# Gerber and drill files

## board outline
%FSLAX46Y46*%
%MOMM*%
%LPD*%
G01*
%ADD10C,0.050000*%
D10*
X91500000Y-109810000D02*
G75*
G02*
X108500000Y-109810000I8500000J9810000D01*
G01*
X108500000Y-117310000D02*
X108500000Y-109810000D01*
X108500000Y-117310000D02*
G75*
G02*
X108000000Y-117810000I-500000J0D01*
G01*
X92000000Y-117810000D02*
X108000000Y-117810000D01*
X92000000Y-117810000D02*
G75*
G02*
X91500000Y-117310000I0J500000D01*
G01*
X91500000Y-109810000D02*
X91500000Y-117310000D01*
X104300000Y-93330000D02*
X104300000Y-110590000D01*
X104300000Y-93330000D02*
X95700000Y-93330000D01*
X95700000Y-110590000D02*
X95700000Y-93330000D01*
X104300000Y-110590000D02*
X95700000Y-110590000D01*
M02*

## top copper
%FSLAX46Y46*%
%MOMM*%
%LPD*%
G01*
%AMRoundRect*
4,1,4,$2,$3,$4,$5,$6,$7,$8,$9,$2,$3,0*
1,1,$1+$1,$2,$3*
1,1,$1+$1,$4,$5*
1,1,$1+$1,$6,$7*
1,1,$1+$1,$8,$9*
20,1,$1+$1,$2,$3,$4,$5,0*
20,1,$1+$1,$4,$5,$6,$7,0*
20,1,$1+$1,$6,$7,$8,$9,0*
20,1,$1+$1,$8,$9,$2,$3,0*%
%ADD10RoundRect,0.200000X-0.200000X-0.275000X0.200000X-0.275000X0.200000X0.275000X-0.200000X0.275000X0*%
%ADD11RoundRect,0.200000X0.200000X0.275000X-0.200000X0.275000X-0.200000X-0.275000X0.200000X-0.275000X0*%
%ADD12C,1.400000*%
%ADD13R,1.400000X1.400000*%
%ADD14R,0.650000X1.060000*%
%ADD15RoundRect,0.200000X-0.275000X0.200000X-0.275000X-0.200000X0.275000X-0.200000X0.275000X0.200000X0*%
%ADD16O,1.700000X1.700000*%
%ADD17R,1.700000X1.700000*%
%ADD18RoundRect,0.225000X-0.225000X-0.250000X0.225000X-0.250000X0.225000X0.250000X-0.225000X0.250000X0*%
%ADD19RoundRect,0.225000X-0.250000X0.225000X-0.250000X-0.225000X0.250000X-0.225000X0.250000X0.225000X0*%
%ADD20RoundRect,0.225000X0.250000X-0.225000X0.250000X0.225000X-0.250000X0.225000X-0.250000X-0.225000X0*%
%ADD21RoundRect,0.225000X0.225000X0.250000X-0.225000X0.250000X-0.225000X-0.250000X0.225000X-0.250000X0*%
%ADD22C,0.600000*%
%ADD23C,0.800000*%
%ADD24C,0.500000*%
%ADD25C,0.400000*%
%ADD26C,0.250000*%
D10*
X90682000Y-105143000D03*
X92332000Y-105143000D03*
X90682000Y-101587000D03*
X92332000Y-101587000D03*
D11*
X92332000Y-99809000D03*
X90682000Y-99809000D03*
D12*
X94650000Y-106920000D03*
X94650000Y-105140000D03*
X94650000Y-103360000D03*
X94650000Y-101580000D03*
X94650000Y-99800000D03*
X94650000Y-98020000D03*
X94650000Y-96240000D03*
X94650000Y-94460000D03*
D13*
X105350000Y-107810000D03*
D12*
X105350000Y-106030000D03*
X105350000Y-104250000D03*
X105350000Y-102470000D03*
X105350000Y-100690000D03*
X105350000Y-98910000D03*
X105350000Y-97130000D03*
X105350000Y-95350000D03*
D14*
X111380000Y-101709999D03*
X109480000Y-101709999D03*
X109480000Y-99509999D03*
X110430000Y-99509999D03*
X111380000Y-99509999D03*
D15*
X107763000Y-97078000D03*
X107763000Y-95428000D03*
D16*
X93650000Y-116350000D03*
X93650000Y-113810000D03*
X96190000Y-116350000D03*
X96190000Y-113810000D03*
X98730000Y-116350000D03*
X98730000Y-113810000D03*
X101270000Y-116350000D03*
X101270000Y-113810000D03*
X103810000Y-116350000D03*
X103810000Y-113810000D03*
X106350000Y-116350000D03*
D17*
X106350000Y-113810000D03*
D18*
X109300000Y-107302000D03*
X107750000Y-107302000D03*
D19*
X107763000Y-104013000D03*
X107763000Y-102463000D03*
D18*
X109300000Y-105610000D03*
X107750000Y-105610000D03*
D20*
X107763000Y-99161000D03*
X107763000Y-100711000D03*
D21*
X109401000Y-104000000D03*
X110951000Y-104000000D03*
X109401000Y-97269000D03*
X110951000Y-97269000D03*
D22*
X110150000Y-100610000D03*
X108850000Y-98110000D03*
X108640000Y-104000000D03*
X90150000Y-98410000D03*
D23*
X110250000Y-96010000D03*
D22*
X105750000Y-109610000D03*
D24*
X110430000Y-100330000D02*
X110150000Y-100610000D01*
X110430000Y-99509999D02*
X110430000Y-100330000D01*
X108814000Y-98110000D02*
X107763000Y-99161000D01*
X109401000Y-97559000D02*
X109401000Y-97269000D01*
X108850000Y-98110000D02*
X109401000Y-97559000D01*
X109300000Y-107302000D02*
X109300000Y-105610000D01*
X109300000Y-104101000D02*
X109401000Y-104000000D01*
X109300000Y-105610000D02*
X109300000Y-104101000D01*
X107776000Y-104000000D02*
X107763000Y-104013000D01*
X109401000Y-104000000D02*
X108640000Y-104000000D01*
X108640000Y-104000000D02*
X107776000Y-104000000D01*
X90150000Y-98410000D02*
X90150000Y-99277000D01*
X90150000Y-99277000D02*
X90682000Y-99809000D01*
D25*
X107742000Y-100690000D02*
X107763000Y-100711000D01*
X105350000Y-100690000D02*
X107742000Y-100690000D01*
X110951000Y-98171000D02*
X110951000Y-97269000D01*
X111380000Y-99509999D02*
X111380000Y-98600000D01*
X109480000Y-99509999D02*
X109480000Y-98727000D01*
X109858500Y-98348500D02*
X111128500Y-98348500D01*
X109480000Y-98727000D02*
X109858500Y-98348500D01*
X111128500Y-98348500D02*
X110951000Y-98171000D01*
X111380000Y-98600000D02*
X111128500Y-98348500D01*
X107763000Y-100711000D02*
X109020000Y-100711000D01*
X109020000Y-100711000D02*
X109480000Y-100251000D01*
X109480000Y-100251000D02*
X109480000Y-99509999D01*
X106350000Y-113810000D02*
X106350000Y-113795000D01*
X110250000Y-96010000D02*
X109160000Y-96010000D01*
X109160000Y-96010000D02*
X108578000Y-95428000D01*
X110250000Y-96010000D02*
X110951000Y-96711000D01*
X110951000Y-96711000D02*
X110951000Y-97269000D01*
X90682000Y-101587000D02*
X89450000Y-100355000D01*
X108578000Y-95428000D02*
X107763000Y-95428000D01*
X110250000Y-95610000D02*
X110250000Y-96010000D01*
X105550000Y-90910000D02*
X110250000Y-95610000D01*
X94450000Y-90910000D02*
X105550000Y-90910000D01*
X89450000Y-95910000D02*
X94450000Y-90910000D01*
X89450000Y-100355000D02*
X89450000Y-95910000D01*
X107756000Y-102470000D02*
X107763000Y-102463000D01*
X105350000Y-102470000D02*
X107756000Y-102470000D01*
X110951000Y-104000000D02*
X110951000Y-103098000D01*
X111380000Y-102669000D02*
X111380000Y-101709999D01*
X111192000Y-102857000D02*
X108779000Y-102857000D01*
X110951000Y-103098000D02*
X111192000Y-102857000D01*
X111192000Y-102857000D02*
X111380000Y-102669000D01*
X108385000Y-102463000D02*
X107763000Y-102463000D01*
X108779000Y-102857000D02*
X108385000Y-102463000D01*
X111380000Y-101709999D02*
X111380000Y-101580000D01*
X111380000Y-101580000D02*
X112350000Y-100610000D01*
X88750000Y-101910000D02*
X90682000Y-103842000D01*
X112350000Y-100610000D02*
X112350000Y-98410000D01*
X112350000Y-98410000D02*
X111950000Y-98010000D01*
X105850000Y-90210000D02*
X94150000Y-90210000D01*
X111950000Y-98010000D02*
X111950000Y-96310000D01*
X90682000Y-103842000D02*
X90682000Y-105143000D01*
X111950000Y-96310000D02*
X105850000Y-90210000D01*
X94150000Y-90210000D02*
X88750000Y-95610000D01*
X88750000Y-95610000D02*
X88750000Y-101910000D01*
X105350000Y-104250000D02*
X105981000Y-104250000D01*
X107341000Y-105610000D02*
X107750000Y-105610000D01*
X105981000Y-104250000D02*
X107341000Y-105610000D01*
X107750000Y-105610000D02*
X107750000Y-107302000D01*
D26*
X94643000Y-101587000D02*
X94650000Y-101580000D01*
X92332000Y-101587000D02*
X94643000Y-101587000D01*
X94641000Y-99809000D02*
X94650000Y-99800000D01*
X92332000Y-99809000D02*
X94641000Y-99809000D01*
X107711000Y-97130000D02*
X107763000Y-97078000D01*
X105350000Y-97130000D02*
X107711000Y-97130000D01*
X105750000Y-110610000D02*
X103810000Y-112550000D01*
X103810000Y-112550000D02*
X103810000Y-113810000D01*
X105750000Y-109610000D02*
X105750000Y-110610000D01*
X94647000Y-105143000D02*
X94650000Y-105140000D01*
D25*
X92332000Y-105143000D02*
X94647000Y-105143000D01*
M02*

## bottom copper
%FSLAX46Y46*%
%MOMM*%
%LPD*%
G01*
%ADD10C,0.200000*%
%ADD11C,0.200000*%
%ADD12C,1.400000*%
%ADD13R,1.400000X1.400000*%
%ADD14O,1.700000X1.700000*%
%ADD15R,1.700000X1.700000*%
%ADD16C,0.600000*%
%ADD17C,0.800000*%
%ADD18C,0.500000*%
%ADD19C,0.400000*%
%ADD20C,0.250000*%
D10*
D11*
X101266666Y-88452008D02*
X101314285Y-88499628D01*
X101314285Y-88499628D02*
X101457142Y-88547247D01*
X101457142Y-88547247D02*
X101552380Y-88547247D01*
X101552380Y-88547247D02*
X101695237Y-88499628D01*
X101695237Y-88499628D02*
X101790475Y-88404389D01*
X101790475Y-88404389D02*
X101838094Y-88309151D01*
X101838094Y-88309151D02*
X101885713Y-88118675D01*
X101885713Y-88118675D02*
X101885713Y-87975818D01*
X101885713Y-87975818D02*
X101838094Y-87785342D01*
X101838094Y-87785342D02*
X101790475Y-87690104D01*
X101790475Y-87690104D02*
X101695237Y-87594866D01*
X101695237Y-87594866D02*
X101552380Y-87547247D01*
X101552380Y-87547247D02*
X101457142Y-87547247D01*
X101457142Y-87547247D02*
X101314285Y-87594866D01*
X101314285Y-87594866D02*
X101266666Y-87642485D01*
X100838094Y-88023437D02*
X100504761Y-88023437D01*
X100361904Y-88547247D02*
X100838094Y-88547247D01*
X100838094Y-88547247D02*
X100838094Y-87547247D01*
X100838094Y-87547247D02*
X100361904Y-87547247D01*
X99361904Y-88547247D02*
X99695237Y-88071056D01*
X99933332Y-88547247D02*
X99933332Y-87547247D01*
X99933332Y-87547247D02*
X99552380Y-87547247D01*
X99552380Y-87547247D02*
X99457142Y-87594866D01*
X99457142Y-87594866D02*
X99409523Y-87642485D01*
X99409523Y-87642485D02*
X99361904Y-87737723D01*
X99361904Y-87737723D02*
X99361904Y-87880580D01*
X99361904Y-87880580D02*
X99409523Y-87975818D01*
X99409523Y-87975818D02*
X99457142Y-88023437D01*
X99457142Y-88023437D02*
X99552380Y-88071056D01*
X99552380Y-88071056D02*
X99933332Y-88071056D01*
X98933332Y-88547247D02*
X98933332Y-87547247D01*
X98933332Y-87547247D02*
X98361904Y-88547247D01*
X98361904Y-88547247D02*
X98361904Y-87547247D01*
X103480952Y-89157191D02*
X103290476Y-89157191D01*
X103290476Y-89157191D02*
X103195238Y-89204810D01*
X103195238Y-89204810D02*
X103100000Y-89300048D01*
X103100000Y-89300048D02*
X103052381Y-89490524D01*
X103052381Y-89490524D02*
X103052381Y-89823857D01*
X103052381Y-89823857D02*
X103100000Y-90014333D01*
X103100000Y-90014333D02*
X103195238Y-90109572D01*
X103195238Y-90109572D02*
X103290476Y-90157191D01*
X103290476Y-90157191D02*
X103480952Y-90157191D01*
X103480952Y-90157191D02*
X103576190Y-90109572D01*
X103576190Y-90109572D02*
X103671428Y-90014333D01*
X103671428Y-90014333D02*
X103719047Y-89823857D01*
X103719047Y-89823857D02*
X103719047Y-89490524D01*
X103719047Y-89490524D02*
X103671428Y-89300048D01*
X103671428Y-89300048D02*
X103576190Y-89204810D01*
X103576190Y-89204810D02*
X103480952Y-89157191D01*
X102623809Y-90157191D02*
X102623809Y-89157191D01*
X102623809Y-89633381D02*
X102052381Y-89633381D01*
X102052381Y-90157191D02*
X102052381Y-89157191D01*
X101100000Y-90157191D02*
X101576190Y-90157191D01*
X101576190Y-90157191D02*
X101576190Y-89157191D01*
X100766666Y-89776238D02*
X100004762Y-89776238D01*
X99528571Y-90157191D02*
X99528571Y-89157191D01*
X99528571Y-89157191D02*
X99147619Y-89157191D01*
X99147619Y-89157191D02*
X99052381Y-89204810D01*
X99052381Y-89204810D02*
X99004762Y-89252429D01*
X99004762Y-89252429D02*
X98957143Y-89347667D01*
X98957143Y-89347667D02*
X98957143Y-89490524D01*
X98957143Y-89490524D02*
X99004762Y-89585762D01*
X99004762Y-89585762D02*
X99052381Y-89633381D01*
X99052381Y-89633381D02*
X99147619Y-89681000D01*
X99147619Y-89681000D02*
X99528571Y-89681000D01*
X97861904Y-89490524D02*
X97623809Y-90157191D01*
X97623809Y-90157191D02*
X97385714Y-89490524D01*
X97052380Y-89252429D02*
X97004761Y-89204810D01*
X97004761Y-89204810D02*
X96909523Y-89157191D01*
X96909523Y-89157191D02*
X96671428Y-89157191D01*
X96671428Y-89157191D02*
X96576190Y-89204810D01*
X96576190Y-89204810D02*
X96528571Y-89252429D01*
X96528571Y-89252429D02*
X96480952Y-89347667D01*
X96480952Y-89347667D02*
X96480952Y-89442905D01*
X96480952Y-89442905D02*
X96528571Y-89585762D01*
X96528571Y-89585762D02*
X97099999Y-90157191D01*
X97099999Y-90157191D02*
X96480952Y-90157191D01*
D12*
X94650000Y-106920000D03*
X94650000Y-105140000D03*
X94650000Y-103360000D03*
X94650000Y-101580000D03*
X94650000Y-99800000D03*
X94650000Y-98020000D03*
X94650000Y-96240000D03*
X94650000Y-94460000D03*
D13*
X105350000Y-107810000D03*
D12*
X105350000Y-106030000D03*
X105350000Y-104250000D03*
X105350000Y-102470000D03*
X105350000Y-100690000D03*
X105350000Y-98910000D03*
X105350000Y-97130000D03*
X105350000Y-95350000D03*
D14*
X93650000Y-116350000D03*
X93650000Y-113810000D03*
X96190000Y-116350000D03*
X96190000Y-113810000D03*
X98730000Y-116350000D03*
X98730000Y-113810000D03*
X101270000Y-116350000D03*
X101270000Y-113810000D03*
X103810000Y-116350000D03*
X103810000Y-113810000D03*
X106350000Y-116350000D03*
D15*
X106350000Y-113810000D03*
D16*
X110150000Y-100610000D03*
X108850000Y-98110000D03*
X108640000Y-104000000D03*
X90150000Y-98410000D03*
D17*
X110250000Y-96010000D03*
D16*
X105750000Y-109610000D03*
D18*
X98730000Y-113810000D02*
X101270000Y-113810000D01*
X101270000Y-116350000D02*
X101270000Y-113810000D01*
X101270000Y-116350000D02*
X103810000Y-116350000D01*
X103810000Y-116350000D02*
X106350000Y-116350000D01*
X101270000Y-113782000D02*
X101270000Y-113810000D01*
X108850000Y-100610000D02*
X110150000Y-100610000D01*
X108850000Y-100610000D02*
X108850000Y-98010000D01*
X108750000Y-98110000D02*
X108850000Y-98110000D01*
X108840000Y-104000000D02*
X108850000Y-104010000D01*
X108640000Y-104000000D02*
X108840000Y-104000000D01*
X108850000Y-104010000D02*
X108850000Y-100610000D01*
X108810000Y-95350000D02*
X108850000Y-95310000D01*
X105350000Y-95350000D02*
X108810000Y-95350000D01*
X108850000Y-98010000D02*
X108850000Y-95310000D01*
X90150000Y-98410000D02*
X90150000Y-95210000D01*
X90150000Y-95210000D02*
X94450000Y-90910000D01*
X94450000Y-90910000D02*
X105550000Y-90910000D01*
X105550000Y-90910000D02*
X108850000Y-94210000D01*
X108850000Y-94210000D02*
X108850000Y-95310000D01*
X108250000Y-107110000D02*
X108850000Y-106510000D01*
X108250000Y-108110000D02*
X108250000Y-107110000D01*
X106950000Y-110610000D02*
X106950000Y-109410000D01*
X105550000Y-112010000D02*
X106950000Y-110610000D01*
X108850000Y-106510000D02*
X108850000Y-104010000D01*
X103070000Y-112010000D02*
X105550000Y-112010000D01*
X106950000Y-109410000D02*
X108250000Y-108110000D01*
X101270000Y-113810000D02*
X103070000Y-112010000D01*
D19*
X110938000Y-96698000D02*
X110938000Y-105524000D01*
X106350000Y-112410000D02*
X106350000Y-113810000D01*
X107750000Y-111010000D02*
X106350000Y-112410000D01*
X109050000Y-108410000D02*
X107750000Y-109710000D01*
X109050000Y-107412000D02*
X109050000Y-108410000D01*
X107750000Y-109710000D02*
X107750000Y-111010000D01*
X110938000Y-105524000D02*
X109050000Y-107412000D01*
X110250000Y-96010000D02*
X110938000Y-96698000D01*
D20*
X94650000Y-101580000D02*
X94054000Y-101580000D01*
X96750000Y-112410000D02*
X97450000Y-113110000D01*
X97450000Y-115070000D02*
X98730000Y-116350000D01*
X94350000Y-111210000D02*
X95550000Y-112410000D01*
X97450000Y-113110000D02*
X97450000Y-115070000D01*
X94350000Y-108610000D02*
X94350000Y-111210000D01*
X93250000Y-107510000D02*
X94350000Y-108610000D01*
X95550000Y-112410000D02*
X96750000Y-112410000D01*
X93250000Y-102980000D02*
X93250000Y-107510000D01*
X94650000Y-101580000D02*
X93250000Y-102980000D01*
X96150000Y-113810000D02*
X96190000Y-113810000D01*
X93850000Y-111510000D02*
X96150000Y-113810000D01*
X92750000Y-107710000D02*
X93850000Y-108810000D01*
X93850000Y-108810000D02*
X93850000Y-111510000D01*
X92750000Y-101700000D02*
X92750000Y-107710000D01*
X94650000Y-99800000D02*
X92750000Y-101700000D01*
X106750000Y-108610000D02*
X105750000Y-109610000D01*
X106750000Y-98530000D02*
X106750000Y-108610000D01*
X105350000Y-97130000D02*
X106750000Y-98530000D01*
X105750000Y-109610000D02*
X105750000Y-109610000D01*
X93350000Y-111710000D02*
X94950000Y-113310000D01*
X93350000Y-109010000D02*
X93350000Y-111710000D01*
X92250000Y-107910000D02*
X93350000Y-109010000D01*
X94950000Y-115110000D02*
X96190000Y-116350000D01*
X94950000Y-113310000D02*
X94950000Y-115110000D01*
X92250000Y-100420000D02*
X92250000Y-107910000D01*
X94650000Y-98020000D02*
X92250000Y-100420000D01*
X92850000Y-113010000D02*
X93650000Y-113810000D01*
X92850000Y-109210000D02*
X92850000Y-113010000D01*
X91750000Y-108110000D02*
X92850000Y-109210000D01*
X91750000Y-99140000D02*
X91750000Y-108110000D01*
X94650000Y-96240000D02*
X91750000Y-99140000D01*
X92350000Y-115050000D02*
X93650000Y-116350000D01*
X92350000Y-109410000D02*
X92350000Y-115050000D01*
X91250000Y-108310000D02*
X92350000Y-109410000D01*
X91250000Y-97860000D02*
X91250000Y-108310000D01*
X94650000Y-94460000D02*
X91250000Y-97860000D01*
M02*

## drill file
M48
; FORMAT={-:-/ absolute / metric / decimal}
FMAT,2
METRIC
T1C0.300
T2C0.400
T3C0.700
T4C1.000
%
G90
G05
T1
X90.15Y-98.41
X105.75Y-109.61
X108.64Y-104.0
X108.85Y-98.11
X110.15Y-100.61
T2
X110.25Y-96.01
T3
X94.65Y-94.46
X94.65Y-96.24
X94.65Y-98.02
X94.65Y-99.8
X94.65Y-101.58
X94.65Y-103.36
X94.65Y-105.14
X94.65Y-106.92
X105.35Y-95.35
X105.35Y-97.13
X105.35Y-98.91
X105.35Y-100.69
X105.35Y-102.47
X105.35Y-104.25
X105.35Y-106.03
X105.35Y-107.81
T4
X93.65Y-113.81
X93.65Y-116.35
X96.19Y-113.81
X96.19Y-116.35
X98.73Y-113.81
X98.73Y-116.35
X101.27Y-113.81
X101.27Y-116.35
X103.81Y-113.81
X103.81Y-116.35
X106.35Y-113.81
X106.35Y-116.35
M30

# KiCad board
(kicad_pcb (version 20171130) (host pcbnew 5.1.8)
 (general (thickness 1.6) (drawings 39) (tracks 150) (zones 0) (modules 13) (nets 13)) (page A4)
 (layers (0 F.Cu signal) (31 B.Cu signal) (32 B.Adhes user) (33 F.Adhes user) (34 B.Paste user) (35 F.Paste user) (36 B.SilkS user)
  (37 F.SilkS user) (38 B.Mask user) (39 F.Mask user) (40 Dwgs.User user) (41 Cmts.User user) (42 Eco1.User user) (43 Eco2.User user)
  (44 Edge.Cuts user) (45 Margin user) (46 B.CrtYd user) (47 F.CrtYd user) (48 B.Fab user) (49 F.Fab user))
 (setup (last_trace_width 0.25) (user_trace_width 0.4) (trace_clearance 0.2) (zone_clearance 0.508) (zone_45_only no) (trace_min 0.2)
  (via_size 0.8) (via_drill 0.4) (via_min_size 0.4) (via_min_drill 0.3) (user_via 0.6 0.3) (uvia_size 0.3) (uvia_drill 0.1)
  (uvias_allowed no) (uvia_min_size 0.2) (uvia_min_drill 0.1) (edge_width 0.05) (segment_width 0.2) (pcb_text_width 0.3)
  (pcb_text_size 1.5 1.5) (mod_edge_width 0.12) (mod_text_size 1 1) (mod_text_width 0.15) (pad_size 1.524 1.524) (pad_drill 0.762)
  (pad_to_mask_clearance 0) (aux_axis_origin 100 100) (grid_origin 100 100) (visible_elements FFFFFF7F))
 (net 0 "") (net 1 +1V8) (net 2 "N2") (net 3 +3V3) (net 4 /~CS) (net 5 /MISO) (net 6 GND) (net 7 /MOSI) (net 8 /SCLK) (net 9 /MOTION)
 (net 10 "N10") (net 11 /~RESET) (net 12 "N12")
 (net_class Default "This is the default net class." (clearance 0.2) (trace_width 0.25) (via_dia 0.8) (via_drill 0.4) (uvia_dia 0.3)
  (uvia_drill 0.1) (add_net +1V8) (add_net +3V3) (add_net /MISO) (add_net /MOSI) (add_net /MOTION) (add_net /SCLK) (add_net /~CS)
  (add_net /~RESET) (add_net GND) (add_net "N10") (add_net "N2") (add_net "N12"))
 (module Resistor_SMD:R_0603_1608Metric (layer F.Cu) (at 91.507 105.143)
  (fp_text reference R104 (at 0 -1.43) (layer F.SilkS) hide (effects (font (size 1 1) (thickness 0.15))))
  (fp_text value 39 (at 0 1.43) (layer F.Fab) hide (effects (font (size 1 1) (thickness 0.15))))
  (pad 1 smd roundrect (at -0.825 0) (size 0.8 0.95) (layers F.Cu F.Paste F.Mask) (roundrect_rratio 0.25) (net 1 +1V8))
  (pad 2 smd roundrect (at 0.825 0) (size 0.8 0.95) (layers F.Cu F.Paste F.Mask) (roundrect_rratio 0.25) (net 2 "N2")))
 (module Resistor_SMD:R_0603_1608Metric (layer F.Cu) (at 91.507 101.587)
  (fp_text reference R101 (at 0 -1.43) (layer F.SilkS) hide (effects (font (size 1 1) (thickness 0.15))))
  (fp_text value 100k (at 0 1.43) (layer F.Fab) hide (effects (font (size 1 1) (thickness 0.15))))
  (pad 1 smd roundrect (at -0.825 0) (size 0.8 0.95) (layers F.Cu F.Paste F.Mask) (roundrect_rratio 0.25) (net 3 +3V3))
  (pad 2 smd roundrect (at 0.825 0) (size 0.8 0.95) (layers F.Cu F.Paste F.Mask) (roundrect_rratio 0.25) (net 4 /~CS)))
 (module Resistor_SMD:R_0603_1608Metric (layer F.Cu) (at 91.507 99.809 180)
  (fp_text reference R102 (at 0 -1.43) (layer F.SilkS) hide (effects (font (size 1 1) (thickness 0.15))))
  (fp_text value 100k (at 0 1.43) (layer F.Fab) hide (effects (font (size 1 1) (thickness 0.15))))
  (pad 1 smd roundrect (at -0.825 0 180) (size 0.8 0.95) (layers F.Cu F.Paste F.Mask) (roundrect_rratio 0.25) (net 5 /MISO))
  (pad 2 smd roundrect (at 0.825 0 180) (size 0.8 0.95) (layers F.Cu F.Paste F.Mask) (roundrect_rratio 0.25) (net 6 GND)))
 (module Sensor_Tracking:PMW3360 (layer F.Cu) (at 105.35 107.81 180)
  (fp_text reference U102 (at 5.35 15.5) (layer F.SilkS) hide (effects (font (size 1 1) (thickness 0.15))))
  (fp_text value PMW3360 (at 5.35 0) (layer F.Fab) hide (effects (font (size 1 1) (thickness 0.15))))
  (fp_line (start 1.05 14.48) (end 1.05 -2.78) (layer Edge.Cuts) (width 0.05))
  (fp_line (start 1.05 14.48) (end 9.65 14.48) (layer Edge.Cuts) (width 0.05))
  (fp_line (start 9.65 -2.78) (end 9.65 14.48) (layer Edge.Cuts) (width 0.05))
  (fp_line (start 1.05 -2.78) (end 9.65 -2.78) (layer Edge.Cuts) (width 0.05))
  (pad 16 thru_hole circle (at 10.7 0.89 180) (size 1.4 1.4) (drill 0.7) (layers *.Cu *.Mask))
  (pad 15 thru_hole circle (at 10.7 2.67 180) (size 1.4 1.4) (drill 0.7) (layers *.Cu *.Mask) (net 2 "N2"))
  (pad 14 thru_hole circle (at 10.7 4.45 180) (size 1.4 1.4) (drill 0.7) (layers *.Cu *.Mask))
  (pad 13 thru_hole circle (at 10.7 6.23 180) (size 1.4 1.4) (drill 0.7) (layers *.Cu *.Mask) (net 4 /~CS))
  (pad 12 thru_hole circle (at 10.7 8.01 180) (size 1.4 1.4) (drill 0.7) (layers *.Cu *.Mask) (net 5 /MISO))
  (pad 11 thru_hole circle (at 10.7 9.79 180) (size 1.4 1.4) (drill 0.7) (layers *.Cu *.Mask) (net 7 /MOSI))
  (pad 10 thru_hole circle (at 10.7 11.57 180) (size 1.4 1.4) (drill 0.7) (layers *.Cu *.Mask) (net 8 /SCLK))
  (pad 9 thru_hole circle (at 10.7 13.35 180) (size 1.4 1.4) (drill 0.7) (layers *.Cu *.Mask) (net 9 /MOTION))
  (pad 1 thru_hole rect (at 0 0 180) (size 1.4 1.4) (drill 0.7) (layers *.Cu *.Mask))
  (pad 2 thru_hole circle (at 0 1.78 180) (size 1.4 1.4) (drill 0.7) (layers *.Cu *.Mask))
  (pad 3 thru_hole circle (at 0 3.56 180) (size 1.4 1.4) (drill 0.7) (layers *.Cu *.Mask) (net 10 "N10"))
  (pad 4 thru_hole circle (at 0 5.34 180) (size 1.4 1.4) (drill 0.7) (layers *.Cu *.Mask) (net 1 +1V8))
  (pad 5 thru_hole circle (at 0 7.12 180) (size 1.4 1.4) (drill 0.7) (layers *.Cu *.Mask) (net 3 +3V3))
  (pad 6 thru_hole circle (at 0 8.9 180) (size 1.4 1.4) (drill 0.7) (layers *.Cu *.Mask))
  (pad 7 thru_hole circle (at 0 10.68 180) (size 1.4 1.4) (drill 0.7) (layers *.Cu *.Mask) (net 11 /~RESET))
  (pad 8 thru_hole circle (at 0 12.46 180) (size 1.4 1.4) (drill 0.7) (layers *.Cu *.Mask) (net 6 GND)))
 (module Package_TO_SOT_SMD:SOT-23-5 (layer F.Cu) (at 110.43 100.609999 270)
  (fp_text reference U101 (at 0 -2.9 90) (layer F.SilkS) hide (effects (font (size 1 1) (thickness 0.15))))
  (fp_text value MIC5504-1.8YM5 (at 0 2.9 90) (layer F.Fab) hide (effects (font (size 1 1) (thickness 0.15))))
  (pad 5 smd rect (at 1.1 -0.95 270) (size 1.06 0.65) (layers F.Cu F.Paste F.Mask) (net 1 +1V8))
  (pad 4 smd rect (at 1.1 0.95 270) (size 1.06 0.65) (layers F.Cu F.Paste F.Mask) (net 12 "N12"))
  (pad 3 smd rect (at -1.1 0.95 270) (size 1.06 0.65) (layers F.Cu F.Paste F.Mask) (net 3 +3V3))
  (pad 2 smd rect (at -1.1 0 270) (size 1.06 0.65) (layers F.Cu F.Paste F.Mask) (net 6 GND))
  (pad 1 smd rect (at -1.1 -0.95 270) (size 1.06 0.65) (layers F.Cu F.Paste F.Mask) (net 3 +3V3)))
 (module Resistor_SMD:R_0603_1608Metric (layer F.Cu) (at 107.763 96.253 270)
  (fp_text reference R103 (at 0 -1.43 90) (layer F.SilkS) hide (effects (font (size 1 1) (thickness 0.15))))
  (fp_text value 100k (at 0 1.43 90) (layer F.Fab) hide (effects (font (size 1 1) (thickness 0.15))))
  (pad 2 smd roundrect (at 0.825 0 270) (size 0.8 0.95) (layers F.Cu F.Paste F.Mask) (roundrect_rratio 0.25) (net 11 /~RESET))
  (pad 1 smd roundrect (at -0.825 0 270) (size 0.8 0.95) (layers F.Cu F.Paste F.Mask) (roundrect_rratio 0.25) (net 3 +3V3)))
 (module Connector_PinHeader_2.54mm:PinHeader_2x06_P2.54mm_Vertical (layer F.Cu) (at 106.35 113.81 270)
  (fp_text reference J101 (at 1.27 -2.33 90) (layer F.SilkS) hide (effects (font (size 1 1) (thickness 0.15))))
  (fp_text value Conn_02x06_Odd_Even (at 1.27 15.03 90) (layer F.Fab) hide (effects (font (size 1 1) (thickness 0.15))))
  (pad 12 thru_hole oval (at 2.54 12.7 270) (size 1.7 1.7) (drill 1) (layers *.Cu *.Mask) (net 9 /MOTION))
  (pad 11 thru_hole oval (at 0 12.7 270) (size 1.7 1.7) (drill 1) (layers *.Cu *.Mask) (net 8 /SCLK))
  (pad 10 thru_hole oval (at 2.54 10.16 270) (size 1.7 1.7) (drill 1) (layers *.Cu *.Mask) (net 7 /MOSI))
  (pad 9 thru_hole oval (at 0 10.16 270) (size 1.7 1.7) (drill 1) (layers *.Cu *.Mask) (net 5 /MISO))
  (pad 8 thru_hole oval (at 2.54 7.62 270) (size 1.7 1.7) (drill 1) (layers *.Cu *.Mask) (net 4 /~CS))
  (pad 7 thru_hole oval (at 0 7.62 270) (size 1.7 1.7) (drill 1) (layers *.Cu *.Mask) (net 6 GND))
  (pad 6 thru_hole oval (at 2.54 5.08 270) (size 1.7 1.7) (drill 1) (layers *.Cu *.Mask) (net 6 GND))
  (pad 5 thru_hole oval (at 0 5.08 270) (size 1.7 1.7) (drill 1) (layers *.Cu *.Mask) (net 6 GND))
  (pad 4 thru_hole oval (at 2.54 2.54 270) (size 1.7 1.7) (drill 1) (layers *.Cu *.Mask) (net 6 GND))
  (pad 3 thru_hole oval (at 0 2.54 270) (size 1.7 1.7) (drill 1) (layers *.Cu *.Mask) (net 11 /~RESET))
  (pad 2 thru_hole oval (at 2.54 0 270) (size 1.7 1.7) (drill 1) (layers *.Cu *.Mask) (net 6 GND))
  (pad 1 thru_hole rect (at 0 0 270) (size 1.7 1.7) (drill 1) (layers *.Cu *.Mask) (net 3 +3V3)))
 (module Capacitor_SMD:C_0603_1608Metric (layer F.Cu) (at 108.525 107.302)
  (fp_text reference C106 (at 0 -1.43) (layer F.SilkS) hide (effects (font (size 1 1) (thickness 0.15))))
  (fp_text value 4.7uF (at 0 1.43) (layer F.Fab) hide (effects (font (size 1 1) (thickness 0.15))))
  (pad 2 smd roundrect (at 0.775 0) (size 0.9 0.95) (layers F.Cu F.Paste F.Mask) (roundrect_rratio 0.25) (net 6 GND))
  (pad 1 smd roundrect (at -0.775 0) (size 0.9 0.95) (layers F.Cu F.Paste F.Mask) (roundrect_rratio 0.25) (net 10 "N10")))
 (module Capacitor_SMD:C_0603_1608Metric (layer F.Cu) (at 107.763 103.238 270)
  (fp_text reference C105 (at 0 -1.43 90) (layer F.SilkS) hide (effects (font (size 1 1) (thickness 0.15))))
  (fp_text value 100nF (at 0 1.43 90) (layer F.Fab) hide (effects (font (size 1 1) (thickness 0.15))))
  (pad 2 smd roundrect (at 0.775 0 270) (size 0.9 0.95) (layers F.Cu F.Paste F.Mask) (roundrect_rratio 0.25) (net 6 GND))
  (pad 1 smd roundrect (at -0.775 0 270) (size 0.9 0.95) (layers F.Cu F.Paste F.Mask) (roundrect_rratio 0.25) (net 1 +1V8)))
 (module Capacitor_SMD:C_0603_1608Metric (layer F.Cu) (at 108.525 105.61)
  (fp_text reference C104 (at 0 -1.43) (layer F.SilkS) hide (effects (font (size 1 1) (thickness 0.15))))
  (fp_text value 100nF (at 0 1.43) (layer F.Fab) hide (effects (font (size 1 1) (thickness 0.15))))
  (pad 2 smd roundrect (at 0.775 0) (size 0.9 0.95) (layers F.Cu F.Paste F.Mask) (roundrect_rratio 0.25) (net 6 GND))
  (pad 1 smd roundrect (at -0.775 0) (size 0.9 0.95) (layers F.Cu F.Paste F.Mask) (roundrect_rratio 0.25) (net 10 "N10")))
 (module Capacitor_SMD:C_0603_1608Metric (layer F.Cu) (at 107.763 99.936 90)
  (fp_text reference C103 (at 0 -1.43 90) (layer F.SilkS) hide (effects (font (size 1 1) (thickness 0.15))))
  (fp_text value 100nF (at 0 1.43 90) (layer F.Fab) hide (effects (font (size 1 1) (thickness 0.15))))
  (pad 2 smd roundrect (at 0.775 0 90) (size 0.9 0.95) (layers F.Cu F.Paste F.Mask) (roundrect_rratio 0.25) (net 6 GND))
  (pad 1 smd roundrect (at -0.775 0 90) (size 0.9 0.95) (layers F.Cu F.Paste F.Mask) (roundrect_rratio 0.25) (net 3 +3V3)))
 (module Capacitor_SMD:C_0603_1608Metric (layer F.Cu) (at 110.176 104 180)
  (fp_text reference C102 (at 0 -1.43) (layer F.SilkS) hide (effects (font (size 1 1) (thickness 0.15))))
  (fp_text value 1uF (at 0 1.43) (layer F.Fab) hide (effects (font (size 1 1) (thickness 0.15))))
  (pad 2 smd roundrect (at 0.775 0 180) (size 0.9 0.95) (layers F.Cu F.Paste F.Mask) (roundrect_rratio 0.25) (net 6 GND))
  (pad 1 smd roundrect (at -0.775 0 180) (size 0.9 0.95) (layers F.Cu F.Paste F.Mask) (roundrect_rratio 0.25) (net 1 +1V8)))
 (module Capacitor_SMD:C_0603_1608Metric (layer F.Cu) (at 110.176 97.269 180)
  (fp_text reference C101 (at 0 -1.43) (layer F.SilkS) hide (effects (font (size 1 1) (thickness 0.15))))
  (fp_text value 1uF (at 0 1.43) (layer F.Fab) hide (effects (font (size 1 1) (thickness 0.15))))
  (pad 2 smd roundrect (at 0.775 0 180) (size 0.9 0.95) (layers F.Cu F.Paste F.Mask) (roundrect_rratio 0.25) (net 6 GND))
  (pad 1 smd roundrect (at -0.775 0 180) (size 0.9 0.95) (layers F.Cu F.Paste F.Mask) (roundrect_rratio 0.25) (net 3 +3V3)))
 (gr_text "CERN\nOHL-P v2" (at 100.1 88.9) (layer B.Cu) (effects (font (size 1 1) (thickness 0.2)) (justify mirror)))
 (gr_arc (start 100 100) (end 108.5 109.81) (angle -278.1845763) (layer Edge.Cuts) (width 0.05))
 (gr_line (start 108.5 117.31) (end 108.5 109.81) (layer Edge.Cuts) (width 0.05))
 (gr_arc (start 108 117.31) (end 108 117.81) (angle -90) (layer Edge.Cuts) (width 0.05))
 (gr_line (start 92 117.81) (end 108 117.81) (layer Edge.Cuts) (width 0.05))
 (gr_arc (start 92 117.31) (end 91.5 117.31) (angle -90) (layer Edge.Cuts) (width 0.05))
 (gr_line (start 91.5 109.81) (end 91.5 117.31) (layer Edge.Cuts) (width 0.05))
 (segment (start 98.73 113.81) (end 101.27 113.81) (width 0.5) (layer B.Cu) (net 6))
 (segment (start 101.27 116.35) (end 101.27 113.81) (width 0.5) (layer B.Cu) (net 6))
 (segment (start 101.27 116.35) (end 103.81 116.35) (width 0.5) (layer B.Cu) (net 6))
 (segment (start 103.81 116.35) (end 106.35 116.35) (width 0.5) (layer B.Cu) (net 6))
 (segment (start 101.27 113.782) (end 101.27 113.81) (width 0.5) (layer B.Cu) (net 6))
 (via (at 110.15 100.61) (size 0.6) (drill 0.3) (layers F.Cu B.Cu) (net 6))
 (segment (start 110.43 100.33) (end 110.15 100.61) (width 0.5) (layer F.Cu) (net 6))
 (segment (start 110.43 99.509999) (end 110.43 100.33) (width 0.5) (layer F.Cu) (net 6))
 (segment (start 108.85 100.61) (end 110.15 100.61) (width 0.5) (layer B.Cu) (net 6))
 (segment (start 108.85 100.61) (end 108.85 98.01) (width 0.5) (layer B.Cu) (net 6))
 (segment (start 108.75 98.11) (end 108.85 98.11) (width 0.5) (layer B.Cu) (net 6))
 (segment (start 108.814 98.11) (end 107.763 99.161) (width 0.5) (layer F.Cu) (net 6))
 (via (at 108.85 98.11) (size 0.6) (drill 0.3) (layers F.Cu B.Cu) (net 6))
 (segment (start 109.401 97.559) (end 109.401 97.269) (width 0.5) (layer F.Cu) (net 6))
 (segment (start 108.85 98.11) (end 109.401 97.559) (width 0.5) (layer F.Cu) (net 6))
 (segment (start 109.3 107.302) (end 109.3 105.61) (width 0.5) (layer F.Cu) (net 6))
 (segment (start 109.3 104.101) (end 109.401 104) (width 0.5) (layer F.Cu) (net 6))
 (segment (start 109.3 105.61) (end 109.3 104.101) (width 0.5) (layer F.Cu) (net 6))
 (segment (start 107.776 104) (end 107.763 104.013) (width 0.5) (layer F.Cu) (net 6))
 (via (at 108.64 104) (size 0.6) (drill 0.3) (layers F.Cu B.Cu) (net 6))
 (segment (start 109.401 104) (end 108.64 104) (width 0.5) (layer F.Cu) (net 6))
 (segment (start 108.64 104) (end 107.776 104) (width 0.5) (layer F.Cu) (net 6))
 (segment (start 108.84 104) (end 108.85 104.01) (width 0.5) (layer B.Cu) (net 6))
 (segment (start 108.64 104) (end 108.84 104) (width 0.5) (layer B.Cu) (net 6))
 (segment (start 108.85 104.01) (end 108.85 100.61) (width 0.5) (layer B.Cu) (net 6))
 (segment (start 108.81 95.35) (end 108.85 95.31) (width 0.5) (layer B.Cu) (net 6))
 (segment (start 105.35 95.35) (end 108.81 95.35) (width 0.5) (layer B.Cu) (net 6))
 (segment (start 108.85 98.01) (end 108.85 95.31) (width 0.5) (layer B.Cu) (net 6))
 (segment (start 90.15 98.41) (end 90.15 99.277) (width 0.5) (layer F.Cu) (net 6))
 (segment (start 90.15 98.41) (end 90.15 95.21) (width 0.5) (layer B.Cu) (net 6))
 (segment (start 90.15 95.21) (end 94.45 90.91) (width 0.5) (layer B.Cu) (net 6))
 (segment (start 94.45 90.91) (end 105.55 90.91) (width 0.5) (layer B.Cu) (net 6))
 (segment (start 105.55 90.91) (end 108.85 94.21) (width 0.5) (layer B.Cu) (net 6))
 (segment (start 108.85 94.21) (end 108.85 95.31) (width 0.5) (layer B.Cu) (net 6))
 (via (at 90.15 98.41) (size 0.6) (drill 0.3) (layers F.Cu B.Cu) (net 6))
 (segment (start 90.15 99.277) (end 90.682 99.809) (width 0.5) (layer F.Cu) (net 6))
 (segment (start 108.25 107.11) (end 108.85 106.51) (width 0.5) (layer B.Cu) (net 6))
 (segment (start 108.25 108.11) (end 108.25 107.11) (width 0.5) (layer B.Cu) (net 6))
 (segment (start 106.95 110.61) (end 106.95 109.41) (width 0.5) (layer B.Cu) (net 6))
 (segment (start 105.55 112.01) (end 106.95 110.61) (width 0.5) (layer B.Cu) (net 6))
 (segment (start 108.85 106.51) (end 108.85 104.01) (width 0.5) (layer B.Cu) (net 6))
 (segment (start 103.07 112.01) (end 105.55 112.01) (width 0.5) (layer B.Cu) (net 6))
 (segment (start 106.95 109.41) (end 108.25 108.11) (width 0.5) (layer B.Cu) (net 6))
 (segment (start 101.27 113.81) (end 103.07 112.01) (width 0.5) (layer B.Cu) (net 6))
 (segment (start 107.742 100.69) (end 107.763 100.711) (width 0.4) (layer F.Cu) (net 3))
 (segment (start 105.35 100.69) (end 107.742 100.69) (width 0.4) (layer F.Cu) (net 3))
 (segment (start 110.951 98.171) (end 110.951 97.269) (width 0.4) (layer F.Cu) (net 3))
 (segment (start 111.38 99.509999) (end 111.38 98.6) (width 0.4) (layer F.Cu) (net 3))
 (segment (start 109.48 99.509999) (end 109.48 98.727) (width 0.4) (layer F.Cu) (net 3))
 (segment (start 109.8585 98.3485) (end 111.1285 98.3485) (width 0.4) (layer F.Cu) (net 3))
 (segment (start 109.48 98.727) (end 109.8585 98.3485) (width 0.4) (layer F.Cu) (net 3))
 (segment (start 111.1285 98.3485) (end 110.951 98.171) (width 0.4) (layer F.Cu) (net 3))
 (segment (start 111.38 98.6) (end 111.1285 98.3485) (width 0.4) (layer F.Cu) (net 3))
 (segment (start 107.763 100.711) (end 109.02 100.711) (width 0.4) (layer F.Cu) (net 3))
 (segment (start 109.02 100.711) (end 109.48 100.251) (width 0.4) (layer F.Cu) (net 3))
 (segment (start 109.48 100.251) (end 109.48 99.509999) (width 0.4) (layer F.Cu) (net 3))
 (segment (start 106.35 113.81) (end 106.35 113.795) (width 0.4) (layer F.Cu) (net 3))
 (segment (start 110.25 96.01) (end 109.16 96.01) (width 0.4) (layer F.Cu) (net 3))
 (segment (start 110.938 96.698) (end 110.938 105.524) (width 0.4) (layer B.Cu) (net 3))
 (segment (start 109.16 96.01) (end 108.578 95.428) (width 0.4) (layer F.Cu) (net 3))
 (segment (start 106.35 112.41) (end 106.35 113.81) (width 0.4) (layer B.Cu) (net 3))
 (segment (start 107.75 111.01) (end 106.35 112.41) (width 0.4) (layer B.Cu) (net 3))
 (segment (start 110.25 96.01) (end 110.951 96.711) (width 0.4) (layer F.Cu) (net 3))
 (segment (start 109.05 108.41) (end 107.75 109.71) (width 0.4) (layer B.Cu) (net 3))
 (segment (start 109.05 107.412) (end 109.05 108.41) (width 0.4) (layer B.Cu) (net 3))
 (segment (start 107.75 109.71) (end 107.75 111.01) (width 0.4) (layer B.Cu) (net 3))
 (segment (start 110.951 96.711) (end 110.951 97.269) (width 0.4) (layer F.Cu) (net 3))
 (segment (start 110.938 105.524) (end 109.05 107.412) (width 0.4) (layer B.Cu) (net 3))
 (via (at 110.25 96.01) (size 0.8) (drill 0.4) (layers F.Cu B.Cu) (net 3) (status 1000000))
 (segment (start 90.682 101.587) (end 89.45 100.355) (width 0.4) (layer F.Cu) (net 3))
 (segment (start 110.25 96.01) (end 110.938 96.698) (width 0.4) (layer B.Cu) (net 3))
 (segment (start 108.578 95.428) (end 107.763 95.428) (width 0.4) (layer F.Cu) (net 3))
 (segment (start 110.25 95.61) (end 110.25 96.01) (width 0.4) (layer F.Cu) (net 3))
 (segment (start 105.55 90.91) (end 110.25 95.61) (width 0.4) (layer F.Cu) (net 3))
 (segment (start 94.45 90.91) (end 105.55 90.91) (width 0.4) (layer F.Cu) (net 3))
 (segment (start 89.45 95.91) (end 94.45 90.91) (width 0.4) (layer F.Cu) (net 3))
 (segment (start 89.45 100.355) (end 89.45 95.91) (width 0.4) (layer F.Cu) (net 3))
 (segment (start 107.756 102.47) (end 107.763 102.463) (width 0.4) (layer F.Cu) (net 1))
 (segment (start 105.35 102.47) (end 107.756 102.47) (width 0.4) (layer F.Cu) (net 1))
 (segment (start 110.951 104) (end 110.951 103.098) (width 0.4) (layer F.Cu) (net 1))
 (segment (start 111.38 102.669) (end 111.38 101.709999) (width 0.4) (layer F.Cu) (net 1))
 (segment (start 111.192 102.857) (end 108.779 102.857) (width 0.4) (layer F.Cu) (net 1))
 (segment (start 110.951 103.098) (end 111.192 102.857) (width 0.4) (layer F.Cu) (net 1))
 (segment (start 111.192 102.857) (end 111.38 102.669) (width 0.4) (layer F.Cu) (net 1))
 (segment (start 108.385 102.463) (end 107.763 102.463) (width 0.4) (layer F.Cu) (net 1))
 (segment (start 108.779 102.857) (end 108.385 102.463) (width 0.4) (layer F.Cu) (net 1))
 (segment (start 111.38 101.709999) (end 111.38 101.58) (width 0.4) (layer F.Cu) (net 1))
 (segment (start 111.38 101.58) (end 112.35 100.61) (width 0.4) (layer F.Cu) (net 1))
 (segment (start 88.75 101.91) (end 90.682 103.842) (width 0.4) (layer F.Cu) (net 1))
 (segment (start 112.35 100.61) (end 112.35 98.41) (width 0.4) (layer F.Cu) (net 1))
 (segment (start 112.35 98.41) (end 111.95 98.01) (width 0.4) (layer F.Cu) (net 1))
 (segment (start 105.85 90.21) (end 94.15 90.21) (width 0.4) (layer F.Cu) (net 1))
 (segment (start 111.95 98.01) (end 111.95 96.31) (width 0.4) (layer F.Cu) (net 1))
 (segment (start 90.682 103.842) (end 90.682 105.143) (width 0.4) (layer F.Cu) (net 1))
 (segment (start 111.95 96.31) (end 105.85 90.21) (width 0.4) (layer F.Cu) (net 1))
 (segment (start 94.15 90.21) (end 88.75 95.61) (width 0.4) (layer F.Cu) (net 1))
 (segment (start 88.75 95.61) (end 88.75 101.91) (width 0.4) (layer F.Cu) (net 1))
 (segment (start 105.35 104.25) (end 105.981 104.25) (width 0.4) (layer F.Cu) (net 10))
 (segment (start 107.341 105.61) (end 107.75 105.61) (width 0.4) (layer F.Cu) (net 10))
 (segment (start 105.981 104.25) (end 107.341 105.61) (width 0.4) (layer F.Cu) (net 10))
 (segment (start 107.75 105.61) (end 107.75 107.302) (width 0.4) (layer F.Cu) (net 10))
 (segment (start 94.643 101.587) (end 94.65 101.58) (width 0.25) (layer F.Cu) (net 4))
 (segment (start 92.332 101.587) (end 94.643 101.587) (width 0.25) (layer F.Cu) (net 4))
 (segment (start 94.65 101.58) (end 94.054 101.58) (width 0.25) (layer B.Cu) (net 4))
 (segment (start 96.75 112.41) (end 97.45 113.11) (width 0.25) (layer B.Cu) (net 4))
 (segment (start 97.45 115.07) (end 98.73 116.35) (width 0.25) (layer B.Cu) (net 4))
 (segment (start 94.35 111.21) (end 95.55 112.41) (width 0.25) (layer B.Cu) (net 4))
 (segment (start 97.45 113.11) (end 97.45 115.07) (width 0.25) (layer B.Cu) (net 4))
 (segment (start 94.35 108.61) (end 94.35 111.21) (width 0.25) (layer B.Cu) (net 4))
 (segment (start 93.25 107.51) (end 94.35 108.61) (width 0.25) (layer B.Cu) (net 4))
 (segment (start 95.55 112.41) (end 96.75 112.41) (width 0.25) (layer B.Cu) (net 4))
 (segment (start 93.25 102.98) (end 93.25 107.51) (width 0.25) (layer B.Cu) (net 4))
 (segment (start 94.65 101.58) (end 93.25 102.98) (width 0.25) (layer B.Cu) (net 4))
 (segment (start 94.641 99.809) (end 94.65 99.8) (width 0.25) (layer F.Cu) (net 5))
 (segment (start 92.332 99.809) (end 94.641 99.809) (width 0.25) (layer F.Cu) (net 5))
 (segment (start 96.15 113.81) (end 96.19 113.81) (width 0.25) (layer B.Cu) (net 5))
 (segment (start 93.85 111.51) (end 96.15 113.81) (width 0.25) (layer B.Cu) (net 5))
 (segment (start 92.75 107.71) (end 93.85 108.81) (width 0.25) (layer B.Cu) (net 5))
 (segment (start 93.85 108.81) (end 93.85 111.51) (width 0.25) (layer B.Cu) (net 5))
 (segment (start 92.75 101.7) (end 92.75 107.71) (width 0.25) (layer B.Cu) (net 5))
 (segment (start 94.65 99.8) (end 92.75 101.7) (width 0.25) (layer B.Cu) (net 5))
 (segment (start 107.711 97.13) (end 107.763 97.078) (width 0.25) (layer F.Cu) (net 11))
 (segment (start 105.35 97.13) (end 107.711 97.13) (width 0.25) (layer F.Cu) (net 11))
 (segment (start 105.75 110.61) (end 103.81 112.55) (width 0.25) (layer F.Cu) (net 11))
 (via (at 105.75 109.61) (size 0.6) (drill 0.3) (layers F.Cu B.Cu) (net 11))
 (segment (start 103.81 112.55) (end 103.81 113.81) (width 0.25) (layer F.Cu) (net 11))
 (segment (start 105.75 109.61) (end 105.75 110.61) (width 0.25) (layer F.Cu) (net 11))
 (segment (start 106.75 108.61) (end 105.75 109.61) (width 0.25) (layer B.Cu) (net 11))
 (segment (start 106.75 98.53) (end 106.75 108.61) (width 0.25) (layer B.Cu) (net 11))
 (segment (start 105.35 97.13) (end 106.75 98.53) (width 0.25) (layer B.Cu) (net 11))
 (segment (start 105.75 109.61) (end 105.75 109.61) (width 0.25) (layer B.Cu) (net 11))
 (segment (start 94.647 105.143) (end 94.65 105.14) (width 0.25) (layer F.Cu) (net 2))
 (segment (start 92.332 105.143) (end 94.647 105.143) (width 0.4) (layer F.Cu) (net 2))
 (segment (start 93.35 111.71) (end 94.95 113.31) (width 0.25) (layer B.Cu) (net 7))
 (segment (start 93.35 109.01) (end 93.35 111.71) (width 0.25) (layer B.Cu) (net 7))
 (segment (start 92.25 107.91) (end 93.35 109.01) (width 0.25) (layer B.Cu) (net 7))
 (segment (start 94.95 115.11) (end 96.19 116.35) (width 0.25) (layer B.Cu) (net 7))
 (segment (start 94.95 113.31) (end 94.95 115.11) (width 0.25) (layer B.Cu) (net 7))
 (segment (start 92.25 100.42) (end 92.25 107.91) (width 0.25) (layer B.Cu) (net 7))
 (segment (start 94.65 98.02) (end 92.25 100.42) (width 0.25) (layer B.Cu) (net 7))
 (segment (start 92.85 113.01) (end 93.65 113.81) (width 0.25) (layer B.Cu) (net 8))
 (segment (start 92.85 109.21) (end 92.85 113.01) (width 0.25) (layer B.Cu) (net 8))
 (segment (start 91.75 108.11) (end 92.85 109.21) (width 0.25) (layer B.Cu) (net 8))
 (segment (start 91.75 99.14) (end 91.75 108.11) (width 0.25) (layer B.Cu) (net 8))
 (segment (start 94.65 96.24) (end 91.75 99.14) (width 0.25) (layer B.Cu) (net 8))
 (segment (start 92.35 115.05) (end 93.65 116.35) (width 0.25) (layer B.Cu) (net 9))
 (segment (start 92.35 109.41) (end 92.35 115.05) (width 0.25) (layer B.Cu) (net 9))
 (segment (start 91.25 108.31) (end 92.35 109.41) (width 0.25) (layer B.Cu) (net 9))
 (segment (start 91.25 97.86) (end 91.25 108.31) (width 0.25) (layer B.Cu) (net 9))
 (segment (start 94.65 94.46) (end 91.25 97.86) (width 0.25) (layer B.Cu) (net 9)))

